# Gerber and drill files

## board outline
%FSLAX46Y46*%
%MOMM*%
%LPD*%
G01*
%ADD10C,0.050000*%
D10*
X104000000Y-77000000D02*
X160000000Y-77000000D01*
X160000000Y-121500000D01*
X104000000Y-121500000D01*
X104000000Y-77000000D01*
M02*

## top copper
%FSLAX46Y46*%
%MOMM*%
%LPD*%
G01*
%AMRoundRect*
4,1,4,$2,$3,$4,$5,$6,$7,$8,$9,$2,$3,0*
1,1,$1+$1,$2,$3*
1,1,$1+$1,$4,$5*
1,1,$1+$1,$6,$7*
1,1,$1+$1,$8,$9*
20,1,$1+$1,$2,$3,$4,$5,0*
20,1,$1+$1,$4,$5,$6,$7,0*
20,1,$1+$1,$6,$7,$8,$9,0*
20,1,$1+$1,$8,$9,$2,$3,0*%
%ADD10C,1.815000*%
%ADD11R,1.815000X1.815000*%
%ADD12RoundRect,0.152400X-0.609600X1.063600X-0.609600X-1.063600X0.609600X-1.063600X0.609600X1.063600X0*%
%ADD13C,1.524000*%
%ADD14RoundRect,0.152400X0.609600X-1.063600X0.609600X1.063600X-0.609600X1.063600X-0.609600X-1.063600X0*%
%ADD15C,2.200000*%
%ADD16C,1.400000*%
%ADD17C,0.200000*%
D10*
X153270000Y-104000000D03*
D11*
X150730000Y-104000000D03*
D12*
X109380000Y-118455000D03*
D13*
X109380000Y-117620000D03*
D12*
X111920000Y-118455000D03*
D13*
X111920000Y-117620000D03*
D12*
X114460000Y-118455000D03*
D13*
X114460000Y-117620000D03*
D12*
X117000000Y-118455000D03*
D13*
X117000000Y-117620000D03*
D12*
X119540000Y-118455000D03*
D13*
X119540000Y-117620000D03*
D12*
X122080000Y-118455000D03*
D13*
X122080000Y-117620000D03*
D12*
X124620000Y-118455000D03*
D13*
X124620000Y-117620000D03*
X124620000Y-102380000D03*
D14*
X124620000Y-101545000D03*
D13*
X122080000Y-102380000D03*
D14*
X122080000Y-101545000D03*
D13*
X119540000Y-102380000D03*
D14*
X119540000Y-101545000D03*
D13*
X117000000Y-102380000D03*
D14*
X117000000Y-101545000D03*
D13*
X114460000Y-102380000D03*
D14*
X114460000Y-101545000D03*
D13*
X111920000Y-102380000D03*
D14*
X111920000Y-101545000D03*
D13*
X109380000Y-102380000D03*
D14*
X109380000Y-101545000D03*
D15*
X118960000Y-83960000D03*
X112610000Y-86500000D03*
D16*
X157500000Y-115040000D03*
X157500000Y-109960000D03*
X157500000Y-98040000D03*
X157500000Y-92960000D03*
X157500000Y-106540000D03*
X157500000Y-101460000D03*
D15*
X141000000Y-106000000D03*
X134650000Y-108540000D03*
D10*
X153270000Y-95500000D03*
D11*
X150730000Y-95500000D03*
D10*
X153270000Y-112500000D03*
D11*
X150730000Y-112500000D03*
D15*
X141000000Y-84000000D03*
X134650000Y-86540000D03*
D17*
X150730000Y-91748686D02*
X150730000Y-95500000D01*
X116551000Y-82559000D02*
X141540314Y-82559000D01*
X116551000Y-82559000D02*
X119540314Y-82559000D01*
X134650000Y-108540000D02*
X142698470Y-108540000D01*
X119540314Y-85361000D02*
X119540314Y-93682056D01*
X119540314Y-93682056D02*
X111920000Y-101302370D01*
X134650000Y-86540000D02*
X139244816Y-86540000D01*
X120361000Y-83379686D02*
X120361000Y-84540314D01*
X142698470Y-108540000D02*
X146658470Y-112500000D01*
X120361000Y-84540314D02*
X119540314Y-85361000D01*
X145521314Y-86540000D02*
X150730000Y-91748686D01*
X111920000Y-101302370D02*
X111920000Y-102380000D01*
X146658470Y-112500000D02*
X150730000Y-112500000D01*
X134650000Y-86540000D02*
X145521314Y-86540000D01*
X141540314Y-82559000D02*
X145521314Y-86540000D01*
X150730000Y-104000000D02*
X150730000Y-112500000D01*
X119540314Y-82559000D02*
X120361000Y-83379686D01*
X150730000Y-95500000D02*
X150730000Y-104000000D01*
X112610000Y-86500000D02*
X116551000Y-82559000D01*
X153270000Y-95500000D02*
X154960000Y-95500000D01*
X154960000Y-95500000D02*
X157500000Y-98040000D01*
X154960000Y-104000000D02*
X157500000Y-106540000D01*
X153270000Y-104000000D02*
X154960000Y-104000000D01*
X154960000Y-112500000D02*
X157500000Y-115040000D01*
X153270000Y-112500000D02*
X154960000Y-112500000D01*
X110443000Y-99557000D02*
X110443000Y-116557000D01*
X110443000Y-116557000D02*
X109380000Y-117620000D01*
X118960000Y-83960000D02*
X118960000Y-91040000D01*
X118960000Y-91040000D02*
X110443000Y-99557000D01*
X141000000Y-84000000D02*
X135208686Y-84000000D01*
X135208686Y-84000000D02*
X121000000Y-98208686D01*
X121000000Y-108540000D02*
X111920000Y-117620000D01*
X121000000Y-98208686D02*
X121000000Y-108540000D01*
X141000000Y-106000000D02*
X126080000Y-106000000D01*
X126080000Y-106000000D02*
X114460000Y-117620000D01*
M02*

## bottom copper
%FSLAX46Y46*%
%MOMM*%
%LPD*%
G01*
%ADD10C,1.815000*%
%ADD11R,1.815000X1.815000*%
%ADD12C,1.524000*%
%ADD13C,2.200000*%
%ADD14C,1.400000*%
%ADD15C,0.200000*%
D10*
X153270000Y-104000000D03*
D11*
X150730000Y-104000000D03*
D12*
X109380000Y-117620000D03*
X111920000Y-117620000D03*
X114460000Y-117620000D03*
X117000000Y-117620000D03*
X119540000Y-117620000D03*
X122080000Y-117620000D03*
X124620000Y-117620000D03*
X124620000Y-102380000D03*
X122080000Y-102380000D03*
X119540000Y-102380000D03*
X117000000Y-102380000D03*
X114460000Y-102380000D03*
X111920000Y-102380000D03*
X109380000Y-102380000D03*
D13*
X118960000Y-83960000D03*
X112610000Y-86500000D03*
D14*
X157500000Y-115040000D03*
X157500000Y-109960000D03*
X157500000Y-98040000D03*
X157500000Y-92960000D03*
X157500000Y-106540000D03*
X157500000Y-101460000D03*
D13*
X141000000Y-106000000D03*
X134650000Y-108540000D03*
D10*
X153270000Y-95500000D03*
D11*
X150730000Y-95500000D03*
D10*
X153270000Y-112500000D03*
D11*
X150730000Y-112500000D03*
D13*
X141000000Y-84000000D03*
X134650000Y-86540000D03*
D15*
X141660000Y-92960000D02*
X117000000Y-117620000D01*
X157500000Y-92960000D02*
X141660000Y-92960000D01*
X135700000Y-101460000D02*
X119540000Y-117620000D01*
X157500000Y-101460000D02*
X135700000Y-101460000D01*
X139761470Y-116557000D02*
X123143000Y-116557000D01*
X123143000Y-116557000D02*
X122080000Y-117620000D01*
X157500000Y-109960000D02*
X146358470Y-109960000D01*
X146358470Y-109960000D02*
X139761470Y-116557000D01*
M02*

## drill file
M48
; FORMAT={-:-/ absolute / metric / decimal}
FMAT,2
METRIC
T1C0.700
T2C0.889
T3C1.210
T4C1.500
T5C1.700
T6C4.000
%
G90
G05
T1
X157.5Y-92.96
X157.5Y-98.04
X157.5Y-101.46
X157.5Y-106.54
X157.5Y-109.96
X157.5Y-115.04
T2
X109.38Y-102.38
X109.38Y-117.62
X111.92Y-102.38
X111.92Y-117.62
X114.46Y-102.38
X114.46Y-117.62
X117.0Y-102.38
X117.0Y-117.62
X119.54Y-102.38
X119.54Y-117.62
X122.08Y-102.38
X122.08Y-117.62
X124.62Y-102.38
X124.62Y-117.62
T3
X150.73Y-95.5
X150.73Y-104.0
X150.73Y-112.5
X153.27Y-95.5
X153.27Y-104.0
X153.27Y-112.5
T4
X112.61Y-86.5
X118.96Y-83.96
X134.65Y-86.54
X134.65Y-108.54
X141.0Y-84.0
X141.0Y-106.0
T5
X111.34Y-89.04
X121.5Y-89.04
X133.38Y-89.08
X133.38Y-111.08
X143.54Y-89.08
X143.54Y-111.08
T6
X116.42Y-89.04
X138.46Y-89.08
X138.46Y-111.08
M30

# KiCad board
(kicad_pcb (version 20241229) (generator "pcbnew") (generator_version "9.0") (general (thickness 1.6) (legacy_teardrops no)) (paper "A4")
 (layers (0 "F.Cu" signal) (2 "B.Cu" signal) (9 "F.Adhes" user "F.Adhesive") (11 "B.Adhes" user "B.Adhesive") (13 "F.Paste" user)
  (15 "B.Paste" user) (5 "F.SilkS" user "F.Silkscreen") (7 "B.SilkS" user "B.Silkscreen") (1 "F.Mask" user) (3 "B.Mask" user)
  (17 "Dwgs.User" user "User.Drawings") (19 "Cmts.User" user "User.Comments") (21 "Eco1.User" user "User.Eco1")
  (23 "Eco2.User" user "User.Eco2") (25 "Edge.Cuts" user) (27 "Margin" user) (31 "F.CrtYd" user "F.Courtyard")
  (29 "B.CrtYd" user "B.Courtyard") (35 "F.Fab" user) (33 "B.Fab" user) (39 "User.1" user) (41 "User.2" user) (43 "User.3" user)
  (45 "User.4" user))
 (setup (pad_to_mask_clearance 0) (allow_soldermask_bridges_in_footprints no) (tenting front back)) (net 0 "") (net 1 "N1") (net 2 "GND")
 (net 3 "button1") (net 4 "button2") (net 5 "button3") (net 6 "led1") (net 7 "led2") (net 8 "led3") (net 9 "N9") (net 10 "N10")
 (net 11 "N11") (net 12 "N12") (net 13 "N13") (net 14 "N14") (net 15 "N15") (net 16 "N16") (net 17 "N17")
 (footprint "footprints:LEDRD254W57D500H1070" (layer "F.Cu") (at 152 104)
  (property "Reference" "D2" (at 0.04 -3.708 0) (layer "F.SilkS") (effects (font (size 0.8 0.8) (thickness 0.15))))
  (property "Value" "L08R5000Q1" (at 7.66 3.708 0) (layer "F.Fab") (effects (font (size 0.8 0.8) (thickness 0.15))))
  (pad "A" thru_hole circle (at 1.27 0) (size 1.815 1.815) (drill 1.21) (layers "*.Cu" "*.Mask") (remove_unused_layers no) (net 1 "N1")
   (solder_mask_margin 0.102))
  (pad "C" thru_hole rect (at -1.27 0) (size 1.815 1.815) (drill 1.21) (layers "*.Cu" "*.Mask") (remove_unused_layers no) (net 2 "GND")
   (solder_mask_margin 0.102)))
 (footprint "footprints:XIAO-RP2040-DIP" (layer "F.Cu") (at 117 110 90)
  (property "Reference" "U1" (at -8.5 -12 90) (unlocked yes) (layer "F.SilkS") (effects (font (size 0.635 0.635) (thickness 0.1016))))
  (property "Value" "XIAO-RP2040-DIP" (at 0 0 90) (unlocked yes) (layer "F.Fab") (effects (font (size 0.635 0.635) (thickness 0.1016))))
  (pad "1" smd roundrect (at -8.455 -7.62 270) (size 2.432 1.524) (layers "F.Cu" "F.Mask") (roundrect_rratio 0.1) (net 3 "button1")
   (thermal_bridge_angle 45))
  (pad "1" thru_hole circle (at -7.62 -7.62 270) (size 1.524 1.524) (drill 0.889) (layers "*.Cu" "*.Mask") (remove_unused_layers no)
   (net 3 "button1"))
  (pad "2" smd roundrect (at -8.455 -5.08 270) (size 2.432 1.524) (layers "F.Cu" "F.Mask") (roundrect_rratio 0.1) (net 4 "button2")
   (thermal_bridge_angle 45))
  (pad "2" thru_hole circle (at -7.62 -5.08 270) (size 1.524 1.524) (drill 0.889) (layers "*.Cu" "*.Mask") (remove_unused_layers no)
   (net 4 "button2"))
  (pad "3" smd roundrect (at -8.455 -2.54 270) (size 2.432 1.524) (layers "F.Cu" "F.Mask") (roundrect_rratio 0.1) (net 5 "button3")
   (thermal_bridge_angle 45))
  (pad "3" thru_hole circle (at -7.62 -2.54 270) (size 1.524 1.524) (drill 0.889) (layers "*.Cu" "*.Mask") (remove_unused_layers no)
   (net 5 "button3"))
  (pad "4" smd roundrect (at -8.455 0 270) (size 2.432 1.524) (layers "F.Cu" "F.Mask") (roundrect_rratio 0.1) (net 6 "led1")
   (thermal_bridge_angle 45))
  (pad "4" thru_hole circle (at -7.62 0 270) (size 1.524 1.524) (drill 0.889) (layers "*.Cu" "*.Mask") (remove_unused_layers no)
   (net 6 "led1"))
  (pad "5" smd roundrect (at -8.455 2.54 270) (size 2.432 1.524) (layers "F.Cu" "F.Mask") (roundrect_rratio 0.1) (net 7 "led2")
   (thermal_bridge_angle 45))
  (pad "5" thru_hole circle (at -7.62 2.54 270) (size 1.524 1.524) (drill 0.889) (layers "*.Cu" "*.Mask") (remove_unused_layers no)
   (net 7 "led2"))
  (pad "6" smd roundrect (at -8.455 5.08 270) (size 2.432 1.524) (layers "F.Cu" "F.Mask") (roundrect_rratio 0.1) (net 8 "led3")
   (thermal_bridge_angle 45))
  (pad "6" thru_hole circle (at -7.62 5.08 270) (size 1.524 1.524) (drill 0.889) (layers "*.Cu" "*.Mask") (remove_unused_layers no)
   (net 8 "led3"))
  (pad "7" smd roundrect (at -8.455 7.62 270) (size 2.432 1.524) (layers "F.Cu" "F.Mask") (roundrect_rratio 0.1) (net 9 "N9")
   (thermal_bridge_angle 45))
  (pad "7" thru_hole circle (at -7.62 7.62 270) (size 1.524 1.524) (drill 0.889) (layers "*.Cu" "*.Mask") (remove_unused_layers no)
   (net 9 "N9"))
  (pad "8" thru_hole circle (at 7.62 7.62 90) (size 1.524 1.524) (drill 0.889) (layers "*.Cu" "*.Mask") (remove_unused_layers no)
   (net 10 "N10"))
  (pad "8" smd roundrect (at 8.455 7.62 90) (size 2.432 1.524) (layers "F.Cu" "F.Mask") (roundrect_rratio 0.1) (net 10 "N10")
   (thermal_bridge_angle 45))
  (pad "9" thru_hole circle (at 7.62 5.08 90) (size 1.524 1.524) (drill 0.889) (layers "*.Cu" "*.Mask") (remove_unused_layers no)
   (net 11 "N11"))
  (pad "9" smd roundrect (at 8.455 5.08 90) (size 2.432 1.524) (layers "F.Cu" "F.Mask") (roundrect_rratio 0.1) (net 11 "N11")
   (thermal_bridge_angle 45))
  (pad "10" thru_hole circle (at 7.62 2.54 90) (size 1.524 1.524) (drill 0.889) (layers "*.Cu" "*.Mask") (remove_unused_layers no)
   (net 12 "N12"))
  (pad "10" smd roundrect (at 8.455 2.54 90) (size 2.432 1.524) (layers "F.Cu" "F.Mask") (roundrect_rratio 0.1) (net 12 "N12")
   (thermal_bridge_angle 45))
  (pad "11" thru_hole circle (at 7.62 0 90) (size 1.524 1.524) (drill 0.889) (layers "*.Cu" "*.Mask") (remove_unused_layers no)
   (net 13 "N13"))
  (pad "11" smd roundrect (at 8.455 0 90) (size 2.432 1.524) (layers "F.Cu" "F.Mask") (roundrect_rratio 0.1) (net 13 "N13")
   (thermal_bridge_angle 45))
  (pad "12" thru_hole circle (at 7.62 -2.54 90) (size 1.524 1.524) (drill 0.889) (layers "*.Cu" "*.Mask") (remove_unused_layers no)
   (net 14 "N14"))
  (pad "12" smd roundrect (at 8.455 -2.54 90) (size 2.432 1.524) (layers "F.Cu" "F.Mask") (roundrect_rratio 0.1) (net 14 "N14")
   (thermal_bridge_angle 45))
  (pad "13" thru_hole circle (at 7.62 -5.08 90) (size 1.524 1.524) (drill 0.889) (layers "*.Cu" "*.Mask") (remove_unused_layers no)
   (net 2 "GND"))
  (pad "13" smd roundrect (at 8.455 -5.08 90) (size 2.432 1.524) (layers "F.Cu" "F.Mask") (roundrect_rratio 0.1) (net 2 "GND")
   (thermal_bridge_angle 45))
  (pad "14" thru_hole circle (at 7.62 -7.62 90) (size 1.524 1.524) (drill 0.889) (layers "*.Cu" "*.Mask") (remove_unused_layers no)
   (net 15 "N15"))
  (pad "14" smd roundrect (at 8.455 -7.62 90) (size 2.432 1.524) (layers "F.Cu" "F.Mask") (roundrect_rratio 0.1) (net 15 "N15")
   (thermal_bridge_angle 45)))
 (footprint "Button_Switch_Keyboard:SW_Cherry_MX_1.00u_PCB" (layer "F.Cu") (at 118.96 83.96)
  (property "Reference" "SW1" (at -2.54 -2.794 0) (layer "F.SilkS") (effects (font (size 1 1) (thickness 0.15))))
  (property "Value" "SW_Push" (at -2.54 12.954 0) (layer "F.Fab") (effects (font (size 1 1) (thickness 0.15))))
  (pad "" np_thru_hole circle (at -7.62 5.08) (size 1.7 1.7) (drill 1.7) (layers "*.Cu" "*.Mask"))
  (pad "" np_thru_hole circle (at -2.54 5.08) (size 4 4) (drill 4) (layers "*.Cu" "*.Mask"))
  (pad "" np_thru_hole circle (at 2.54 5.08) (size 1.7 1.7) (drill 1.7) (layers "*.Cu" "*.Mask"))
  (pad "1" thru_hole circle (at 0 0) (size 2.2 2.2) (drill 1.5) (layers "*.Cu" "*.Mask") (remove_unused_layers no) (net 3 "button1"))
  (pad "2" thru_hole circle (at -6.35 2.54) (size 2.2 2.2) (drill 1.5) (layers "*.Cu" "*.Mask") (remove_unused_layers no) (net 2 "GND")))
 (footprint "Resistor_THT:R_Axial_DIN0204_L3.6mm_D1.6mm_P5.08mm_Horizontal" (layer "F.Cu") (at 157.5 115.04 90)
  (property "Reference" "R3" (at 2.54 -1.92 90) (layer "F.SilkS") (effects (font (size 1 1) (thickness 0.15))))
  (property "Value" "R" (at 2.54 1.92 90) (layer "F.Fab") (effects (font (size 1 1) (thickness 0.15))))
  (pad "1" thru_hole circle (at 0 0 90) (size 1.4 1.4) (drill 0.7) (layers "*.Cu" "*.Mask") (remove_unused_layers no) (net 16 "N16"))
  (pad "2" thru_hole circle (at 5.08 0 90) (size 1.4 1.4) (drill 0.7) (layers "*.Cu" "*.Mask") (remove_unused_layers no) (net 8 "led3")))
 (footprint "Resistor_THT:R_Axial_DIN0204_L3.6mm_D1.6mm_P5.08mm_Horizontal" (layer "F.Cu") (at 157.5 98.04 90)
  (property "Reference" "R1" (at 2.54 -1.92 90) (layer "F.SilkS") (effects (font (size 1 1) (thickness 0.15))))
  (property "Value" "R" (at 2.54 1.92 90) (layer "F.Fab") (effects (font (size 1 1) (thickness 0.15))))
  (pad "1" thru_hole circle (at 0 0 90) (size 1.4 1.4) (drill 0.7) (layers "*.Cu" "*.Mask") (remove_unused_layers no) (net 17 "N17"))
  (pad "2" thru_hole circle (at 5.08 0 90) (size 1.4 1.4) (drill 0.7) (layers "*.Cu" "*.Mask") (remove_unused_layers no) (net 6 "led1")))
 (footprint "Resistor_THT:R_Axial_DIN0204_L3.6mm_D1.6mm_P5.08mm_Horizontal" (layer "F.Cu") (at 157.5 106.54 90)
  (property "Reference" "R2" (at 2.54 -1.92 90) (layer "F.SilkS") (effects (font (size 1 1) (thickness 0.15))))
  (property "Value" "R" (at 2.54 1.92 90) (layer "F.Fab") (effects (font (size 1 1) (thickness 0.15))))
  (pad "1" thru_hole circle (at 0 0 90) (size 1.4 1.4) (drill 0.7) (layers "*.Cu" "*.Mask") (remove_unused_layers no) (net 1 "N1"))
  (pad "2" thru_hole circle (at 5.08 0 90) (size 1.4 1.4) (drill 0.7) (layers "*.Cu" "*.Mask") (remove_unused_layers no) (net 7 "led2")))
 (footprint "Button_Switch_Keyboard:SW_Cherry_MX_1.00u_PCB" (layer "F.Cu") (at 141 106)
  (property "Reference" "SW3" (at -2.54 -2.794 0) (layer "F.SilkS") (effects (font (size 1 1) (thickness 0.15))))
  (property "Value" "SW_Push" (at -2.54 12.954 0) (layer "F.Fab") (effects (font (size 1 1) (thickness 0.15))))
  (pad "" np_thru_hole circle (at -7.62 5.08) (size 1.7 1.7) (drill 1.7) (layers "*.Cu" "*.Mask"))
  (pad "" np_thru_hole circle (at -2.54 5.08) (size 4 4) (drill 4) (layers "*.Cu" "*.Mask"))
  (pad "" np_thru_hole circle (at 2.54 5.08) (size 1.7 1.7) (drill 1.7) (layers "*.Cu" "*.Mask"))
  (pad "1" thru_hole circle (at 0 0) (size 2.2 2.2) (drill 1.5) (layers "*.Cu" "*.Mask") (remove_unused_layers no) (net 5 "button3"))
  (pad "2" thru_hole circle (at -6.35 2.54) (size 2.2 2.2) (drill 1.5) (layers "*.Cu" "*.Mask") (remove_unused_layers no) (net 2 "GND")))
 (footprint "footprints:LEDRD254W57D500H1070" (layer "F.Cu") (at 152 95.5)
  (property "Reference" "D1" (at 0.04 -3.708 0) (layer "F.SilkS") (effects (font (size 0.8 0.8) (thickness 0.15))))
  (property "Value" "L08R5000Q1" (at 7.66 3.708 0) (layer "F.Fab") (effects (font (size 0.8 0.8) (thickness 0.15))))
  (pad "A" thru_hole circle (at 1.27 0) (size 1.815 1.815) (drill 1.21) (layers "*.Cu" "*.Mask") (remove_unused_layers no) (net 17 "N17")
   (solder_mask_margin 0.102))
  (pad "C" thru_hole rect (at -1.27 0) (size 1.815 1.815) (drill 1.21) (layers "*.Cu" "*.Mask") (remove_unused_layers no) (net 2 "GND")
   (solder_mask_margin 0.102)))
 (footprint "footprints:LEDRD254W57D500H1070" (layer "F.Cu") (at 152 112.5)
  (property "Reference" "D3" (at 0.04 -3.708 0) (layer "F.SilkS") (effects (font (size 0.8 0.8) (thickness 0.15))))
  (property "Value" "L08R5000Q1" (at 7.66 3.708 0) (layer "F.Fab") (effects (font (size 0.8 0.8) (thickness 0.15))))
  (pad "A" thru_hole circle (at 1.27 0) (size 1.815 1.815) (drill 1.21) (layers "*.Cu" "*.Mask") (remove_unused_layers no) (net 16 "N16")
   (solder_mask_margin 0.102))
  (pad "C" thru_hole rect (at -1.27 0) (size 1.815 1.815) (drill 1.21) (layers "*.Cu" "*.Mask") (remove_unused_layers no) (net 2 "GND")
   (solder_mask_margin 0.102)))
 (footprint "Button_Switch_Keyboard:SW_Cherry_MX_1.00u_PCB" (layer "F.Cu") (at 141 84)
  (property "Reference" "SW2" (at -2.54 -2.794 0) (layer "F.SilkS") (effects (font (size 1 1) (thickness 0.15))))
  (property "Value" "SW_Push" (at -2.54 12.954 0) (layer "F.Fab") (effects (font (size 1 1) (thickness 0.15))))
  (pad "" np_thru_hole circle (at -7.62 5.08) (size 1.7 1.7) (drill 1.7) (layers "*.Cu" "*.Mask"))
  (pad "" np_thru_hole circle (at -2.54 5.08) (size 4 4) (drill 4) (layers "*.Cu" "*.Mask"))
  (pad "" np_thru_hole circle (at 2.54 5.08) (size 1.7 1.7) (drill 1.7) (layers "*.Cu" "*.Mask"))
  (pad "1" thru_hole circle (at 0 0) (size 2.2 2.2) (drill 1.5) (layers "*.Cu" "*.Mask") (remove_unused_layers no) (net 4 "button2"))
  (pad "2" thru_hole circle (at -6.35 2.54) (size 2.2 2.2) (drill 1.5) (layers "*.Cu" "*.Mask") (remove_unused_layers no) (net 2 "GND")))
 (gr_rect (start 104 77) (end 160 121.5) (stroke (width 0.05) (type default)) (fill no) (layer "Edge.Cuts"))
 (segment (start 150.73 91.748686) (end 150.73 95.5) (width 0.2) (layer "F.Cu") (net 2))
 (segment (start 116.551 82.559) (end 141.540314 82.559) (width 0.2) (layer "F.Cu") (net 2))
 (segment (start 116.551 82.559) (end 119.540314 82.559) (width 0.2) (layer "F.Cu") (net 2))
 (segment (start 134.65 108.54) (end 142.69847 108.54) (width 0.2) (layer "F.Cu") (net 2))
 (segment (start 119.540314 85.361) (end 119.540314 93.682056) (width 0.2) (layer "F.Cu") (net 2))
 (segment (start 119.540314 93.682056) (end 111.92 101.30237) (width 0.2) (layer "F.Cu") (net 2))
 (segment (start 134.65 86.54) (end 139.244816 86.54) (width 0.2) (layer "F.Cu") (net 2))
 (segment (start 120.361 83.379686) (end 120.361 84.540314) (width 0.2) (layer "F.Cu") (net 2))
 (segment (start 142.69847 108.54) (end 146.65847 112.5) (width 0.2) (layer "F.Cu") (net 2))
 (segment (start 120.361 84.540314) (end 119.540314 85.361) (width 0.2) (layer "F.Cu") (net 2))
 (segment (start 145.521314 86.54) (end 150.73 91.748686) (width 0.2) (layer "F.Cu") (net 2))
 (segment (start 111.92 101.30237) (end 111.92 102.38) (width 0.2) (layer "F.Cu") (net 2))
 (segment (start 146.65847 112.5) (end 150.73 112.5) (width 0.2) (layer "F.Cu") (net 2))
 (segment (start 134.65 86.54) (end 145.521314 86.54) (width 0.2) (layer "F.Cu") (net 2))
 (segment (start 141.540314 82.559) (end 145.521314 86.54) (width 0.2) (layer "F.Cu") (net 2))
 (segment (start 150.73 104) (end 150.73 112.5) (width 0.2) (layer "F.Cu") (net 2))
 (segment (start 119.540314 82.559) (end 120.361 83.379686) (width 0.2) (layer "F.Cu") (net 2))
 (segment (start 150.73 95.5) (end 150.73 104) (width 0.2) (layer "F.Cu") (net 2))
 (segment (start 112.61 86.5) (end 116.551 82.559) (width 0.2) (layer "F.Cu") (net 2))
 (segment (start 153.27 95.5) (end 154.96 95.5) (width 0.2) (layer "F.Cu") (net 17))
 (segment (start 154.96 95.5) (end 157.5 98.04) (width 0.2) (layer "F.Cu") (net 17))
 (segment (start 154.96 104) (end 157.5 106.54) (width 0.2) (layer "F.Cu") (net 1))
 (segment (start 153.27 104) (end 154.96 104) (width 0.2) (layer "F.Cu") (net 1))
 (segment (start 154.96 112.5) (end 157.5 115.04) (width 0.2) (layer "F.Cu") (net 16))
 (segment (start 153.27 112.5) (end 154.96 112.5) (width 0.2) (layer "F.Cu") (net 16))
 (segment (start 141.66 92.96) (end 117 117.62) (width 0.2) (layer "B.Cu") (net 6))
 (segment (start 157.5 92.96) (end 141.66 92.96) (width 0.2) (layer "B.Cu") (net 6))
 (segment (start 135.7 101.46) (end 119.54 117.62) (width 0.2) (layer "B.Cu") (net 7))
 (segment (start 157.5 101.46) (end 135.7 101.46) (width 0.2) (layer "B.Cu") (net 7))
 (segment (start 139.76147 116.557) (end 123.143 116.557) (width 0.2) (layer "B.Cu") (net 8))
 (segment (start 123.143 116.557) (end 122.08 117.62) (width 0.2) (layer "B.Cu") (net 8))
 (segment (start 157.5 109.96) (end 146.35847 109.96) (width 0.2) (layer "B.Cu") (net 8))
 (segment (start 146.35847 109.96) (end 139.76147 116.557) (width 0.2) (layer "B.Cu") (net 8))
 (segment (start 110.443 99.557) (end 110.443 116.557) (width 0.2) (layer "F.Cu") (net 3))
 (segment (start 110.443 116.557) (end 109.38 117.62) (width 0.2) (layer "F.Cu") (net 3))
 (segment (start 118.96 83.96) (end 118.96 91.04) (width 0.2) (layer "F.Cu") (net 3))
 (segment (start 118.96 91.04) (end 110.443 99.557) (width 0.2) (layer "F.Cu") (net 3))
 (segment (start 141 84) (end 135.208686 84) (width 0.2) (layer "F.Cu") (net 4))
 (segment (start 135.208686 84) (end 121 98.208686) (width 0.2) (layer "F.Cu") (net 4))
 (segment (start 121 108.54) (end 111.92 117.62) (width 0.2) (layer "F.Cu") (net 4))
 (segment (start 121 98.208686) (end 121 108.54) (width 0.2) (layer "F.Cu") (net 4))
 (segment (start 141 106) (end 126.08 106) (width 0.2) (layer "F.Cu") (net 5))
 (segment (start 126.08 106) (end 114.46 117.62) (width 0.2) (layer "F.Cu") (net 5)))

